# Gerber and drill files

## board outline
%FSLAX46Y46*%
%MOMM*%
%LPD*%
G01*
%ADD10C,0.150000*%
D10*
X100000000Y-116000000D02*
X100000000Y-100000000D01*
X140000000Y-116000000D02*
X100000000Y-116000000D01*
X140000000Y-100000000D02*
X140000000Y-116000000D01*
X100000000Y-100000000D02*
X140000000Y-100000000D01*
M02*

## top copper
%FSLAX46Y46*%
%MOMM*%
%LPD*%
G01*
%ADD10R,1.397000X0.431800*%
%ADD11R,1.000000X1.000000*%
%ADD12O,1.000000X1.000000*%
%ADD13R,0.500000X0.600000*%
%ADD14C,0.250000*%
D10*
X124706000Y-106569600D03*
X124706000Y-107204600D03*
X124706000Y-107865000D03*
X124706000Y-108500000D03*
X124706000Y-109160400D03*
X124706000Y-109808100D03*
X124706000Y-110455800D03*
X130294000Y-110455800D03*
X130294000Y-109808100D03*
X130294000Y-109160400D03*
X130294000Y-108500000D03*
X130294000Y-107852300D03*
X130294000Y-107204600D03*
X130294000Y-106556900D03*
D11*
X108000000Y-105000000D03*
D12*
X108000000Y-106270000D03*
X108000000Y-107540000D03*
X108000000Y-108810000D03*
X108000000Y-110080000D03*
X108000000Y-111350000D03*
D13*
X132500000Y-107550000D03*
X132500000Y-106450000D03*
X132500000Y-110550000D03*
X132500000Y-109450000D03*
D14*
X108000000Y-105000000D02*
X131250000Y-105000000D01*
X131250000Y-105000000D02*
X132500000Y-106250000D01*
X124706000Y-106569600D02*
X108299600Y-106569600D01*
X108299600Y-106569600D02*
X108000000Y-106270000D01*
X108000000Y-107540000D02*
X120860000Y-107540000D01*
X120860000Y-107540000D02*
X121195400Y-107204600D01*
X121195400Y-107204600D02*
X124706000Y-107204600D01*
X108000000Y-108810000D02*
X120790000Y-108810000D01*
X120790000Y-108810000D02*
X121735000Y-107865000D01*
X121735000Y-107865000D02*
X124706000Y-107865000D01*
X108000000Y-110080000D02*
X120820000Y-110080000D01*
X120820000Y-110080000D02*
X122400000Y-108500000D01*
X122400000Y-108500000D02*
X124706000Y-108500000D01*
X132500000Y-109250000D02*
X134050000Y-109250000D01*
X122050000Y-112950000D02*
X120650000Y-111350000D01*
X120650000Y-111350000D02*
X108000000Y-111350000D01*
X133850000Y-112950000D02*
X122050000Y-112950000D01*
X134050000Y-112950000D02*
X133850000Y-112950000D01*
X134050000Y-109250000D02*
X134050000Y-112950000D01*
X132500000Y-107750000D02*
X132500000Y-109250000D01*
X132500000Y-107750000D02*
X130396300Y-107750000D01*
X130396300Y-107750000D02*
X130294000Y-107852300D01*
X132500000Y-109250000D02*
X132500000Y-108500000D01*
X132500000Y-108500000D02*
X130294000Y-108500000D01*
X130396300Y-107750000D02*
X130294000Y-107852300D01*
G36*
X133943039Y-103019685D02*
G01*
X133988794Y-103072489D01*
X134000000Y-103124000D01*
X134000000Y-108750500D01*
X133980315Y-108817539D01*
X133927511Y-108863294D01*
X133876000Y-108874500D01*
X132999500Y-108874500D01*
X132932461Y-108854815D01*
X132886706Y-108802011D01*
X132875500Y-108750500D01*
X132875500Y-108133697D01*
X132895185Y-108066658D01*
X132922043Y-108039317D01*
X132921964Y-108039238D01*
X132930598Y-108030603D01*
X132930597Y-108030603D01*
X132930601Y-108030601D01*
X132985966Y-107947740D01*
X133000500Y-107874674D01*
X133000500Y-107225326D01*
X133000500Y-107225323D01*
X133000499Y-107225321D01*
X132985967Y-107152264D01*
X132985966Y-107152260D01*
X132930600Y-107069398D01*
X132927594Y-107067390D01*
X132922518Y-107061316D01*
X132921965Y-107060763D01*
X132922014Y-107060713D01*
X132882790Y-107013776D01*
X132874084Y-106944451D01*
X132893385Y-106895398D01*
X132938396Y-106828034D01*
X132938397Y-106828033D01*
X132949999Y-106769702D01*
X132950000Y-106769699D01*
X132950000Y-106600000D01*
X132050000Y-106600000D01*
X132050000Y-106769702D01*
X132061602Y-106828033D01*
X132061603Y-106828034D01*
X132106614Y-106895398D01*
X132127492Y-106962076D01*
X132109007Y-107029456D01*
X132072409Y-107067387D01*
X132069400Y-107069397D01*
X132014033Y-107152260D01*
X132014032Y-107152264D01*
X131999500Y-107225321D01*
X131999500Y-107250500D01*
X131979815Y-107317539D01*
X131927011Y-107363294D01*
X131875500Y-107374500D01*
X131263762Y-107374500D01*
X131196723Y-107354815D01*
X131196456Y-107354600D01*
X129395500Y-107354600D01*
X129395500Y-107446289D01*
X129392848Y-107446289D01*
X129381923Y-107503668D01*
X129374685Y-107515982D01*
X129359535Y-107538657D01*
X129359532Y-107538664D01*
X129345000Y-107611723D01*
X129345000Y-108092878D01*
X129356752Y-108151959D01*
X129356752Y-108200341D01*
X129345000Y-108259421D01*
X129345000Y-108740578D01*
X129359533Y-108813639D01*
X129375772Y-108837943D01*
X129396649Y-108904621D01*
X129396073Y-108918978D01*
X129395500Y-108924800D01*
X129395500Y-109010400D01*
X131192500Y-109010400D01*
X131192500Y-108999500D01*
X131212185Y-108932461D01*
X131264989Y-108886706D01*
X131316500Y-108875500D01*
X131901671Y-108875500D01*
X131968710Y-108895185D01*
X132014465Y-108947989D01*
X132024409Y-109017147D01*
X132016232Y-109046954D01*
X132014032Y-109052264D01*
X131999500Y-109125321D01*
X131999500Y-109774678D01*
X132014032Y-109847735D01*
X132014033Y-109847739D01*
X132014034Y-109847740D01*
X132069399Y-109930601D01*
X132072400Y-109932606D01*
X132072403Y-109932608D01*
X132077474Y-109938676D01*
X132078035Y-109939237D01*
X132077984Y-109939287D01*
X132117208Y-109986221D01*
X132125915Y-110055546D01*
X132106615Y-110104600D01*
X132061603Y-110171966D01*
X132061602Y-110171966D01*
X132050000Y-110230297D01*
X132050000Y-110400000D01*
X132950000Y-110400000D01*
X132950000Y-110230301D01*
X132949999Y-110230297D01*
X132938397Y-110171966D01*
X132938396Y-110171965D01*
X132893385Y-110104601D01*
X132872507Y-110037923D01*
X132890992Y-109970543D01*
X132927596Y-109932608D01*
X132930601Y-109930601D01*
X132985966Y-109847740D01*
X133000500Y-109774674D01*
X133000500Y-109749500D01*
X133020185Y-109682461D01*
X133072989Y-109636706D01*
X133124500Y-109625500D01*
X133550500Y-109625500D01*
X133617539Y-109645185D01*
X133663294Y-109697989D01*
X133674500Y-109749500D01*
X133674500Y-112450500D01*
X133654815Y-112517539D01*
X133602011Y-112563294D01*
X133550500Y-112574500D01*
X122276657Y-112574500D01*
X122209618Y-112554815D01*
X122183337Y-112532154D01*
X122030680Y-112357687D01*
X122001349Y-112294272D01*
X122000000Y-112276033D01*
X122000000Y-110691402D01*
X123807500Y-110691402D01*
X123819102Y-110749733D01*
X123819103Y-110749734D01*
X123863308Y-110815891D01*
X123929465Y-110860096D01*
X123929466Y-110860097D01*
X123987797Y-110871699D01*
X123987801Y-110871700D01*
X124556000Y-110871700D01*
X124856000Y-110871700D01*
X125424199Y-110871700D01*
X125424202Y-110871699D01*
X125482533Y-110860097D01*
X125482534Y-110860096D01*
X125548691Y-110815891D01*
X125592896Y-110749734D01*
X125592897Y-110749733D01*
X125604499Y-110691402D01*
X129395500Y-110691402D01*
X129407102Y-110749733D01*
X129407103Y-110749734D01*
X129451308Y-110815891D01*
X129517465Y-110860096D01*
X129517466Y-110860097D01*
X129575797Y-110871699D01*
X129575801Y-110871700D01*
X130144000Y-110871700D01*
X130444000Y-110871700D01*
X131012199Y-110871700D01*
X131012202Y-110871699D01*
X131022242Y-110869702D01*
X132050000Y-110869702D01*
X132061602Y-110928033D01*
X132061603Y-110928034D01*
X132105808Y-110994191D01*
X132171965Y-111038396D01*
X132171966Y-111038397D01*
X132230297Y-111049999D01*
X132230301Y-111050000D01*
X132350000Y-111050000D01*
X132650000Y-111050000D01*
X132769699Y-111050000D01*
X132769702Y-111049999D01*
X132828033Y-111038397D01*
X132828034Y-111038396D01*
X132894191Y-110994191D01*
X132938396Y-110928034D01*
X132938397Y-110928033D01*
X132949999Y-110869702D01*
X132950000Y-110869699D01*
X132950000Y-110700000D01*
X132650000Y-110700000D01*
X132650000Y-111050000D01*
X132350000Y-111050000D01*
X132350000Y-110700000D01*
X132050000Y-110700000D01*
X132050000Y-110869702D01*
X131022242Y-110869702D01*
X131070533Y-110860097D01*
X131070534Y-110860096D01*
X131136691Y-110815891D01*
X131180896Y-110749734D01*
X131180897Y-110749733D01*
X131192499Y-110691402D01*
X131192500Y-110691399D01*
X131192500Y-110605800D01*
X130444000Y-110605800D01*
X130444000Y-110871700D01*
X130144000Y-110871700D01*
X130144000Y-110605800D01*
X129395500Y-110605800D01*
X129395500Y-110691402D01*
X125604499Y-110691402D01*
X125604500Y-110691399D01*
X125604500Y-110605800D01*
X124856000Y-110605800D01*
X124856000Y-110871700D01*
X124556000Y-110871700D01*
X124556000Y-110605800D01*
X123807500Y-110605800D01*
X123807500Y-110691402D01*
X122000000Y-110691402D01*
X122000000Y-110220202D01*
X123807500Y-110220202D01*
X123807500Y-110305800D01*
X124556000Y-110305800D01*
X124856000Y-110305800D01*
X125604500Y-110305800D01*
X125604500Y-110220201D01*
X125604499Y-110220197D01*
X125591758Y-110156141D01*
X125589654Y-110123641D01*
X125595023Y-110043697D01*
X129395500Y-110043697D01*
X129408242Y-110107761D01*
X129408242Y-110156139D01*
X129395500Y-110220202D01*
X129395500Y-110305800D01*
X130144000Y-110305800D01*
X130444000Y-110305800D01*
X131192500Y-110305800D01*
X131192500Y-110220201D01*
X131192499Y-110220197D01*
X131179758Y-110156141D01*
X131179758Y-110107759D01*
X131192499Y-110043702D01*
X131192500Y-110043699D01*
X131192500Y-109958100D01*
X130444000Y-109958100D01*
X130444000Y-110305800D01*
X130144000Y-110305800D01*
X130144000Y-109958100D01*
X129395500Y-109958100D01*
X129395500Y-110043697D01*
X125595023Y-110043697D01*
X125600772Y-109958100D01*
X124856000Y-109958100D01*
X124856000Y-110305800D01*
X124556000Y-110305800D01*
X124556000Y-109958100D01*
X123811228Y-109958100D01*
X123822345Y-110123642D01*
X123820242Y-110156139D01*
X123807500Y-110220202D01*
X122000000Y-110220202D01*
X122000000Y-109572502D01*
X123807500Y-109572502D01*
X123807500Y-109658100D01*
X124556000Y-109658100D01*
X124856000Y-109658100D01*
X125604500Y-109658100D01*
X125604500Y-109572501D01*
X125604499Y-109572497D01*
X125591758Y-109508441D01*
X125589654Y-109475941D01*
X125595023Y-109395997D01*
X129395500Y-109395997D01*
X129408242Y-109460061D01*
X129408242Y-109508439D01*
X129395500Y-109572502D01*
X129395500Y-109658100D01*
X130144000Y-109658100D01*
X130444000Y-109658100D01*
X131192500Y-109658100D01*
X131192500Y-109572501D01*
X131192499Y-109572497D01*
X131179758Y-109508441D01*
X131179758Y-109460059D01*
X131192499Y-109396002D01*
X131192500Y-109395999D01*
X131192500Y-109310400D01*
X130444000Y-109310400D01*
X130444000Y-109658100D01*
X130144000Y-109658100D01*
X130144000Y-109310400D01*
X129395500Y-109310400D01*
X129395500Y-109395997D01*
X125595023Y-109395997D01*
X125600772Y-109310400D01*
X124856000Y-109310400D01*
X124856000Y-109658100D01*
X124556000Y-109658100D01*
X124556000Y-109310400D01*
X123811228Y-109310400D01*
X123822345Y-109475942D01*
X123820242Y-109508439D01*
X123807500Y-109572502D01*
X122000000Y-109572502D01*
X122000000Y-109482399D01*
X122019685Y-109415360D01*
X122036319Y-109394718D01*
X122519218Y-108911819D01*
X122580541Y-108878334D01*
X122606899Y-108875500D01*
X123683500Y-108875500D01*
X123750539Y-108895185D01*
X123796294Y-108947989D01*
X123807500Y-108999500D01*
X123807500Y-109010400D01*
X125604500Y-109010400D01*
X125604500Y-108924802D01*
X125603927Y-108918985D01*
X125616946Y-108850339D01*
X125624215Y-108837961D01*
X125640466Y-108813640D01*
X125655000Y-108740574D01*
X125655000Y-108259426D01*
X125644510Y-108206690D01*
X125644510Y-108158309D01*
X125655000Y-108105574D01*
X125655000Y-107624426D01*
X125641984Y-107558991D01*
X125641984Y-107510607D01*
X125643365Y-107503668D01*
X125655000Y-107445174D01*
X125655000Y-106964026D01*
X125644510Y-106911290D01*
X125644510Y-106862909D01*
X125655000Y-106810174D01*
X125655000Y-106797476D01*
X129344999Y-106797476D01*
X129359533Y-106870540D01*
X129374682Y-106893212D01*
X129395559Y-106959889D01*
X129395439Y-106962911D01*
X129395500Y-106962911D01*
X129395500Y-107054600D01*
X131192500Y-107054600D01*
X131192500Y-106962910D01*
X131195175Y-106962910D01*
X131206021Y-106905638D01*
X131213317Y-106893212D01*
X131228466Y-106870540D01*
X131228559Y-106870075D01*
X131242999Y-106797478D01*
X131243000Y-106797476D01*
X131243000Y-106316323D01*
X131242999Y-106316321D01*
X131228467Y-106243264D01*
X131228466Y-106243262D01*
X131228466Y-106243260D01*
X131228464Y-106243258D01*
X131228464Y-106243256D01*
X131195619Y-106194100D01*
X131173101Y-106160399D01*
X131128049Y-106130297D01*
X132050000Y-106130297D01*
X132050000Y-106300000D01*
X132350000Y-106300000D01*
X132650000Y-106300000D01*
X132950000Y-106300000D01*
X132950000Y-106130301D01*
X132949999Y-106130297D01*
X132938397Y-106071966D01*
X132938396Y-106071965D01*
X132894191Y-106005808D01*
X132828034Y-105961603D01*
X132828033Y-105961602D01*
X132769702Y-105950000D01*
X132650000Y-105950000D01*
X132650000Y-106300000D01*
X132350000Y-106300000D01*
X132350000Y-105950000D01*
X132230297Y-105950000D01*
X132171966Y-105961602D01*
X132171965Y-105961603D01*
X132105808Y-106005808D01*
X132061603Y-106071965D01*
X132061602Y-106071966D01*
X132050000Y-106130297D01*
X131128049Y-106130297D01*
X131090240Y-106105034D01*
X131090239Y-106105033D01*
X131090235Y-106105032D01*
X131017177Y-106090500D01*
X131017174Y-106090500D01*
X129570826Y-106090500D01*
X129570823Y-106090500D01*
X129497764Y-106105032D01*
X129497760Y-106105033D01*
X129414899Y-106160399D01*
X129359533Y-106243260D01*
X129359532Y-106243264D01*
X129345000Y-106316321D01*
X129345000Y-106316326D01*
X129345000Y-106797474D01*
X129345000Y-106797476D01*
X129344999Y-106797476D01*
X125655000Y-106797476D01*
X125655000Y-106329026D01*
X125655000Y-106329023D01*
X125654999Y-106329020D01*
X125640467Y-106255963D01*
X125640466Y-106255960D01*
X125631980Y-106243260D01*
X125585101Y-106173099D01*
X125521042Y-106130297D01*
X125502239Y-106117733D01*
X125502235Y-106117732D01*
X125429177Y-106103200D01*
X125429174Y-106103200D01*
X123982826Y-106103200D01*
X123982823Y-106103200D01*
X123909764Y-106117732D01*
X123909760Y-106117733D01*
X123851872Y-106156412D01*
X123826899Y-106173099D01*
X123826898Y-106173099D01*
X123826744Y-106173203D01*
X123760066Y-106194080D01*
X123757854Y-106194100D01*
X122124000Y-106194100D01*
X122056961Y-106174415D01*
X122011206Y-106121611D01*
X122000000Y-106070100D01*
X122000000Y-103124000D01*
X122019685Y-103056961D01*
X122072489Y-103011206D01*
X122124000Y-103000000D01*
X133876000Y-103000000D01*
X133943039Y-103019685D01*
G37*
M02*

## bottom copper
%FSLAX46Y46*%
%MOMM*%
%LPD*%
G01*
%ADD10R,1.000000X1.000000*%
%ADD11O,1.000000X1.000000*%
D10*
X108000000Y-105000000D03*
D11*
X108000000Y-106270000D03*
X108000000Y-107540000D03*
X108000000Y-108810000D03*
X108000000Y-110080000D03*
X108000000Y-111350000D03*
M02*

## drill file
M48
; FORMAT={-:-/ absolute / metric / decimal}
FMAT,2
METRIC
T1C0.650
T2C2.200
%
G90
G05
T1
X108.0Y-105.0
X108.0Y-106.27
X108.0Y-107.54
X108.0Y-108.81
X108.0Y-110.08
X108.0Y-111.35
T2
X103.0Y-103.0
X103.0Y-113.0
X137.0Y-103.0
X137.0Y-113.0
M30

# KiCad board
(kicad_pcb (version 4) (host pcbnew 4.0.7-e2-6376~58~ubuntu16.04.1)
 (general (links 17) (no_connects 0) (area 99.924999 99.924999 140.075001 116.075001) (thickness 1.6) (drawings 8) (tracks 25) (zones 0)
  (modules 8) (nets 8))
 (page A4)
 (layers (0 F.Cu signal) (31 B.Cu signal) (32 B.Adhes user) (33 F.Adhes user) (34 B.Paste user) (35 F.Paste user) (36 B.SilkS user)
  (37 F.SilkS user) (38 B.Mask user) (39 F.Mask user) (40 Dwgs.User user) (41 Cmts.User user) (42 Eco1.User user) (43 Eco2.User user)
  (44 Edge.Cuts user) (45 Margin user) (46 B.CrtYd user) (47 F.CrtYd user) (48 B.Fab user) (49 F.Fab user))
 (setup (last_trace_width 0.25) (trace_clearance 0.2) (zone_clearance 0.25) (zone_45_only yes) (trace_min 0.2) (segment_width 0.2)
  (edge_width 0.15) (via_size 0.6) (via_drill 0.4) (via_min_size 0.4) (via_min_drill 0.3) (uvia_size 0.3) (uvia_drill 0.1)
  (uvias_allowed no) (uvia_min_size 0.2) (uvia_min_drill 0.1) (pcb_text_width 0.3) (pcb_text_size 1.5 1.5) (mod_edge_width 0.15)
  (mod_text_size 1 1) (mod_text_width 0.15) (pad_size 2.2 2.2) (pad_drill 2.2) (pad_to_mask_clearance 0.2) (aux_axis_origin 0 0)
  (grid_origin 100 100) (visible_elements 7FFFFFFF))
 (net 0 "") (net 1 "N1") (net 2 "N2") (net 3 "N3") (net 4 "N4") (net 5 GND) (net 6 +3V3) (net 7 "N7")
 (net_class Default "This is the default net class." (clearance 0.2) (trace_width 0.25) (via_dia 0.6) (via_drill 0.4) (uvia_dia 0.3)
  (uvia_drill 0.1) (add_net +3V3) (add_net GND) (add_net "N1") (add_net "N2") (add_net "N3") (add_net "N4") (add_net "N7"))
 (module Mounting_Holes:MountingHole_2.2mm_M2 (layer F.Cu) (at 103 103)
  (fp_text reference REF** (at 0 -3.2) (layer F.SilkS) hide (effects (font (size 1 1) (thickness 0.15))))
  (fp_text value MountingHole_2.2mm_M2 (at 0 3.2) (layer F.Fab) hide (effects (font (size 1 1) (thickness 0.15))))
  (pad 1 np_thru_hole circle (at 0 0) (size 2.2 2.2) (drill 2.2) (layers *.Cu *.Mask)))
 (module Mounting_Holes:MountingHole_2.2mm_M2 (layer F.Cu) (at 103 113)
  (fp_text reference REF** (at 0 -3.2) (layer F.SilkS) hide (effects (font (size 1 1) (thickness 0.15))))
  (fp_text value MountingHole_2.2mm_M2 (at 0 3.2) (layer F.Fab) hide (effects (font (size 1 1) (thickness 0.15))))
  (pad 1 np_thru_hole circle (at 0 0) (size 2.2 2.2) (drill 2.2) (layers *.Cu *.Mask)))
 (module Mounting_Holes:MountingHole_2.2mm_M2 (layer F.Cu) (at 137 113)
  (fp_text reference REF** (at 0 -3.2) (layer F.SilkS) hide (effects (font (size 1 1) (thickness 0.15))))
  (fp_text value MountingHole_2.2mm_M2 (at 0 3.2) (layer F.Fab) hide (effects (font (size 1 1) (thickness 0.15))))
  (pad 1 np_thru_hole circle (at 0 0) (size 2.2 2.2) (drill 2.2) (layers *.Cu *.Mask)))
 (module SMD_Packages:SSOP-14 (layer F.Cu) (at 127.5 108.5 270)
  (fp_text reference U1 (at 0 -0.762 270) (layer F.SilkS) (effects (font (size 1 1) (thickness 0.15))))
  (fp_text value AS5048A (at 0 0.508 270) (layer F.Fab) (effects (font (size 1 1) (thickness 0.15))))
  (pad 1 smd rect (at -1.9304 2.794 270) (size 0.4318 1.397) (layers F.Cu F.Paste F.Mask) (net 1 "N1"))
  (pad 2 smd rect (at -1.2954 2.794 270) (size 0.4318 1.397) (layers F.Cu F.Paste F.Mask) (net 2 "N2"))
  (pad 3 smd rect (at -0.635 2.794 270) (size 0.4318 1.397) (layers F.Cu F.Paste F.Mask) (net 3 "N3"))
  (pad 4 smd rect (at 0 2.794 270) (size 0.4318 1.397) (layers F.Cu F.Paste F.Mask) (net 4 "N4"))
  (pad 5 smd rect (at 0.6604 2.794 270) (size 0.4318 1.397) (layers F.Cu F.Paste F.Mask) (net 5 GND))
  (pad 6 smd rect (at 1.3081 2.794 270) (size 0.4318 1.397) (layers F.Cu F.Paste F.Mask) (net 5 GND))
  (pad 7 smd rect (at 1.9558 2.794 270) (size 0.4318 1.397) (layers F.Cu F.Paste F.Mask) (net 5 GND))
  (pad 8 smd rect (at 1.9558 -2.794 270) (size 0.4318 1.397) (layers F.Cu F.Paste F.Mask) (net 5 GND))
  (pad 9 smd rect (at 1.3081 -2.794 270) (size 0.4318 1.397) (layers F.Cu F.Paste F.Mask) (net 5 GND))
  (pad 10 smd rect (at 0.6604 -2.794 270) (size 0.4318 1.397) (layers F.Cu F.Paste F.Mask) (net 5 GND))
  (pad 11 smd rect (at 0 -2.794 270) (size 0.4318 1.397) (layers F.Cu F.Paste F.Mask) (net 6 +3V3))
  (pad 12 smd rect (at -0.6477 -2.794 270) (size 0.4318 1.397) (layers F.Cu F.Paste F.Mask) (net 6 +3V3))
  (pad 13 smd rect (at -1.2954 -2.794 270) (size 0.4318 1.397) (layers F.Cu F.Paste F.Mask) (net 5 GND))
  (pad 14 smd rect (at -1.9431 -2.794 270) (size 0.4318 1.397) (layers F.Cu F.Paste F.Mask) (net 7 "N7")))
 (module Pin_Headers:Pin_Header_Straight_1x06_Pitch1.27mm (layer F.Cu) (at 108 105)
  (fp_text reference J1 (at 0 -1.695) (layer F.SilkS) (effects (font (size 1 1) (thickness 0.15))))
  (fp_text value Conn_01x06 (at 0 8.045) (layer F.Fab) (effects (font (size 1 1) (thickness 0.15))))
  (pad 1 thru_hole rect (at 0 0) (size 1 1) (drill 0.65) (layers *.Cu *.Mask) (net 5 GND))
  (pad 2 thru_hole oval (at 0 1.27) (size 1 1) (drill 0.65) (layers *.Cu *.Mask) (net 1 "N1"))
  (pad 3 thru_hole oval (at 0 2.54) (size 1 1) (drill 0.65) (layers *.Cu *.Mask) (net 2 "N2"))
  (pad 4 thru_hole oval (at 0 3.81) (size 1 1) (drill 0.65) (layers *.Cu *.Mask) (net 3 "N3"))
  (pad 5 thru_hole oval (at 0 5.08) (size 1 1) (drill 0.65) (layers *.Cu *.Mask) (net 4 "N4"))
  (pad 6 thru_hole oval (at 0 6.35) (size 1 1) (drill 0.65) (layers *.Cu *.Mask) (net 6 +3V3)))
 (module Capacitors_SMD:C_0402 (layer F.Cu) (at 132.5 107 90)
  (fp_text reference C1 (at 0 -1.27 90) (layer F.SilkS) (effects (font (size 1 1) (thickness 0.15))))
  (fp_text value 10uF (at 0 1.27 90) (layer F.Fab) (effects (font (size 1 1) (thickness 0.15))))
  (pad 1 smd rect (at -0.55 0 90) (size 0.6 0.5) (layers F.Cu F.Paste F.Mask) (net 6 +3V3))
  (pad 2 smd rect (at 0.55 0 90) (size 0.6 0.5) (layers F.Cu F.Paste F.Mask) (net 5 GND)))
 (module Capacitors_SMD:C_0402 (layer F.Cu) (at 132.5 110 90)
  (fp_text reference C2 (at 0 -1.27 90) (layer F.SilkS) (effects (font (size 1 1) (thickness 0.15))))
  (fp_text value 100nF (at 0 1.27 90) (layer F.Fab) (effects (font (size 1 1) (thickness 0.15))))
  (pad 1 smd rect (at -0.55 0 90) (size 0.6 0.5) (layers F.Cu F.Paste F.Mask) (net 5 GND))
  (pad 2 smd rect (at 0.55 0 90) (size 0.6 0.5) (layers F.Cu F.Paste F.Mask) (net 6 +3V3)))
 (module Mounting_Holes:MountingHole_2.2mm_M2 (layer F.Cu) (at 137 103)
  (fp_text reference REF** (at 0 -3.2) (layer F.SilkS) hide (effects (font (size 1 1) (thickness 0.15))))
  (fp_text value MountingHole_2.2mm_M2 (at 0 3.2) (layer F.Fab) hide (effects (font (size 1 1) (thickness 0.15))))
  (pad 1 np_thru_hole circle (at 0 0) (size 2.2 2.2) (drill 2.2) (layers *.Cu *.Mask)))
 (gr_line (start 100 116) (end 100 100) (angle 90) (layer Edge.Cuts) (width 0.15))
 (gr_line (start 140 116) (end 100 116) (angle 90) (layer Edge.Cuts) (width 0.15))
 (gr_line (start 140 100) (end 140 116) (angle 90) (layer Edge.Cuts) (width 0.15))
 (gr_line (start 100 100) (end 140 100) (angle 90) (layer Edge.Cuts) (width 0.15))
 (segment (start 108 105) (end 131.25 105) (width 0.25) (layer F.Cu) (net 5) (status 10))
 (segment (start 131.25 105) (end 132.5 106.25) (width 0.25) (layer F.Cu) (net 5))
 (segment (start 124.706 106.5696) (end 108.2996 106.5696) (width 0.25) (layer F.Cu) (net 1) (status 20))
 (segment (start 108.2996 106.5696) (end 108 106.27) (width 0.25) (layer F.Cu) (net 1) (status 30))
 (segment (start 108 107.54) (end 120.86 107.54) (width 0.25) (layer F.Cu) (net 2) (status 10))
 (segment (start 120.86 107.54) (end 121.1954 107.2046) (width 0.25) (layer F.Cu) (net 2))
 (segment (start 121.1954 107.2046) (end 124.706 107.2046) (width 0.25) (layer F.Cu) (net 2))
 (segment (start 108 108.81) (end 120.79 108.81) (width 0.25) (layer F.Cu) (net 3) (status 10))
 (segment (start 120.79 108.81) (end 121.735 107.865) (width 0.25) (layer F.Cu) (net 3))
 (segment (start 121.735 107.865) (end 124.706 107.865) (width 0.25) (layer F.Cu) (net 3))
 (segment (start 108 110.08) (end 120.82 110.08) (width 0.25) (layer F.Cu) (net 4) (status 10))
 (segment (start 120.82 110.08) (end 122.4 108.5) (width 0.25) (layer F.Cu) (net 4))
 (segment (start 122.4 108.5) (end 124.706 108.5) (width 0.25) (layer F.Cu) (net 4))
 (segment (start 132.5 109.25) (end 134.05 109.25) (width 0.25) (layer F.Cu) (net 6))
 (segment (start 122.05 112.95) (end 120.65 111.35) (width 0.25) (layer F.Cu) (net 6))
 (segment (start 120.65 111.35) (end 108 111.35) (width 0.25) (layer F.Cu) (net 6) (status 20))
 (segment (start 133.85 112.95) (end 122.05 112.95) (width 0.25) (layer F.Cu) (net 6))
 (segment (start 134.05 112.95) (end 133.85 112.95) (width 0.25) (layer F.Cu) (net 6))
 (segment (start 134.05 109.25) (end 134.05 112.95) (width 0.25) (layer F.Cu) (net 6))
 (segment (start 132.5 107.75) (end 132.5 109.25) (width 0.25) (layer F.Cu) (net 6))
 (segment (start 132.5 107.75) (end 130.3963 107.75) (width 0.25) (layer F.Cu) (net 6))
 (segment (start 130.3963 107.75) (end 130.294 107.8523) (width 0.25) (layer F.Cu) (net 6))
 (segment (start 132.5 109.25) (end 132.5 108.5) (width 0.25) (layer F.Cu) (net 6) (status 12))
 (segment (start 132.5 108.5) (end 130.294 108.5) (width 0.25) (layer F.Cu) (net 6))
 (segment (start 130.3963 107.75) (end 130.294 107.8523) (width 0.25) (layer F.Cu) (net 6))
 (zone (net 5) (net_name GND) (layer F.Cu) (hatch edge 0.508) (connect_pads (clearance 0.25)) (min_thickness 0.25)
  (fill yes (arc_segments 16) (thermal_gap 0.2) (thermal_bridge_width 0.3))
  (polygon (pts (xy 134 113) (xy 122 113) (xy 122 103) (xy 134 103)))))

